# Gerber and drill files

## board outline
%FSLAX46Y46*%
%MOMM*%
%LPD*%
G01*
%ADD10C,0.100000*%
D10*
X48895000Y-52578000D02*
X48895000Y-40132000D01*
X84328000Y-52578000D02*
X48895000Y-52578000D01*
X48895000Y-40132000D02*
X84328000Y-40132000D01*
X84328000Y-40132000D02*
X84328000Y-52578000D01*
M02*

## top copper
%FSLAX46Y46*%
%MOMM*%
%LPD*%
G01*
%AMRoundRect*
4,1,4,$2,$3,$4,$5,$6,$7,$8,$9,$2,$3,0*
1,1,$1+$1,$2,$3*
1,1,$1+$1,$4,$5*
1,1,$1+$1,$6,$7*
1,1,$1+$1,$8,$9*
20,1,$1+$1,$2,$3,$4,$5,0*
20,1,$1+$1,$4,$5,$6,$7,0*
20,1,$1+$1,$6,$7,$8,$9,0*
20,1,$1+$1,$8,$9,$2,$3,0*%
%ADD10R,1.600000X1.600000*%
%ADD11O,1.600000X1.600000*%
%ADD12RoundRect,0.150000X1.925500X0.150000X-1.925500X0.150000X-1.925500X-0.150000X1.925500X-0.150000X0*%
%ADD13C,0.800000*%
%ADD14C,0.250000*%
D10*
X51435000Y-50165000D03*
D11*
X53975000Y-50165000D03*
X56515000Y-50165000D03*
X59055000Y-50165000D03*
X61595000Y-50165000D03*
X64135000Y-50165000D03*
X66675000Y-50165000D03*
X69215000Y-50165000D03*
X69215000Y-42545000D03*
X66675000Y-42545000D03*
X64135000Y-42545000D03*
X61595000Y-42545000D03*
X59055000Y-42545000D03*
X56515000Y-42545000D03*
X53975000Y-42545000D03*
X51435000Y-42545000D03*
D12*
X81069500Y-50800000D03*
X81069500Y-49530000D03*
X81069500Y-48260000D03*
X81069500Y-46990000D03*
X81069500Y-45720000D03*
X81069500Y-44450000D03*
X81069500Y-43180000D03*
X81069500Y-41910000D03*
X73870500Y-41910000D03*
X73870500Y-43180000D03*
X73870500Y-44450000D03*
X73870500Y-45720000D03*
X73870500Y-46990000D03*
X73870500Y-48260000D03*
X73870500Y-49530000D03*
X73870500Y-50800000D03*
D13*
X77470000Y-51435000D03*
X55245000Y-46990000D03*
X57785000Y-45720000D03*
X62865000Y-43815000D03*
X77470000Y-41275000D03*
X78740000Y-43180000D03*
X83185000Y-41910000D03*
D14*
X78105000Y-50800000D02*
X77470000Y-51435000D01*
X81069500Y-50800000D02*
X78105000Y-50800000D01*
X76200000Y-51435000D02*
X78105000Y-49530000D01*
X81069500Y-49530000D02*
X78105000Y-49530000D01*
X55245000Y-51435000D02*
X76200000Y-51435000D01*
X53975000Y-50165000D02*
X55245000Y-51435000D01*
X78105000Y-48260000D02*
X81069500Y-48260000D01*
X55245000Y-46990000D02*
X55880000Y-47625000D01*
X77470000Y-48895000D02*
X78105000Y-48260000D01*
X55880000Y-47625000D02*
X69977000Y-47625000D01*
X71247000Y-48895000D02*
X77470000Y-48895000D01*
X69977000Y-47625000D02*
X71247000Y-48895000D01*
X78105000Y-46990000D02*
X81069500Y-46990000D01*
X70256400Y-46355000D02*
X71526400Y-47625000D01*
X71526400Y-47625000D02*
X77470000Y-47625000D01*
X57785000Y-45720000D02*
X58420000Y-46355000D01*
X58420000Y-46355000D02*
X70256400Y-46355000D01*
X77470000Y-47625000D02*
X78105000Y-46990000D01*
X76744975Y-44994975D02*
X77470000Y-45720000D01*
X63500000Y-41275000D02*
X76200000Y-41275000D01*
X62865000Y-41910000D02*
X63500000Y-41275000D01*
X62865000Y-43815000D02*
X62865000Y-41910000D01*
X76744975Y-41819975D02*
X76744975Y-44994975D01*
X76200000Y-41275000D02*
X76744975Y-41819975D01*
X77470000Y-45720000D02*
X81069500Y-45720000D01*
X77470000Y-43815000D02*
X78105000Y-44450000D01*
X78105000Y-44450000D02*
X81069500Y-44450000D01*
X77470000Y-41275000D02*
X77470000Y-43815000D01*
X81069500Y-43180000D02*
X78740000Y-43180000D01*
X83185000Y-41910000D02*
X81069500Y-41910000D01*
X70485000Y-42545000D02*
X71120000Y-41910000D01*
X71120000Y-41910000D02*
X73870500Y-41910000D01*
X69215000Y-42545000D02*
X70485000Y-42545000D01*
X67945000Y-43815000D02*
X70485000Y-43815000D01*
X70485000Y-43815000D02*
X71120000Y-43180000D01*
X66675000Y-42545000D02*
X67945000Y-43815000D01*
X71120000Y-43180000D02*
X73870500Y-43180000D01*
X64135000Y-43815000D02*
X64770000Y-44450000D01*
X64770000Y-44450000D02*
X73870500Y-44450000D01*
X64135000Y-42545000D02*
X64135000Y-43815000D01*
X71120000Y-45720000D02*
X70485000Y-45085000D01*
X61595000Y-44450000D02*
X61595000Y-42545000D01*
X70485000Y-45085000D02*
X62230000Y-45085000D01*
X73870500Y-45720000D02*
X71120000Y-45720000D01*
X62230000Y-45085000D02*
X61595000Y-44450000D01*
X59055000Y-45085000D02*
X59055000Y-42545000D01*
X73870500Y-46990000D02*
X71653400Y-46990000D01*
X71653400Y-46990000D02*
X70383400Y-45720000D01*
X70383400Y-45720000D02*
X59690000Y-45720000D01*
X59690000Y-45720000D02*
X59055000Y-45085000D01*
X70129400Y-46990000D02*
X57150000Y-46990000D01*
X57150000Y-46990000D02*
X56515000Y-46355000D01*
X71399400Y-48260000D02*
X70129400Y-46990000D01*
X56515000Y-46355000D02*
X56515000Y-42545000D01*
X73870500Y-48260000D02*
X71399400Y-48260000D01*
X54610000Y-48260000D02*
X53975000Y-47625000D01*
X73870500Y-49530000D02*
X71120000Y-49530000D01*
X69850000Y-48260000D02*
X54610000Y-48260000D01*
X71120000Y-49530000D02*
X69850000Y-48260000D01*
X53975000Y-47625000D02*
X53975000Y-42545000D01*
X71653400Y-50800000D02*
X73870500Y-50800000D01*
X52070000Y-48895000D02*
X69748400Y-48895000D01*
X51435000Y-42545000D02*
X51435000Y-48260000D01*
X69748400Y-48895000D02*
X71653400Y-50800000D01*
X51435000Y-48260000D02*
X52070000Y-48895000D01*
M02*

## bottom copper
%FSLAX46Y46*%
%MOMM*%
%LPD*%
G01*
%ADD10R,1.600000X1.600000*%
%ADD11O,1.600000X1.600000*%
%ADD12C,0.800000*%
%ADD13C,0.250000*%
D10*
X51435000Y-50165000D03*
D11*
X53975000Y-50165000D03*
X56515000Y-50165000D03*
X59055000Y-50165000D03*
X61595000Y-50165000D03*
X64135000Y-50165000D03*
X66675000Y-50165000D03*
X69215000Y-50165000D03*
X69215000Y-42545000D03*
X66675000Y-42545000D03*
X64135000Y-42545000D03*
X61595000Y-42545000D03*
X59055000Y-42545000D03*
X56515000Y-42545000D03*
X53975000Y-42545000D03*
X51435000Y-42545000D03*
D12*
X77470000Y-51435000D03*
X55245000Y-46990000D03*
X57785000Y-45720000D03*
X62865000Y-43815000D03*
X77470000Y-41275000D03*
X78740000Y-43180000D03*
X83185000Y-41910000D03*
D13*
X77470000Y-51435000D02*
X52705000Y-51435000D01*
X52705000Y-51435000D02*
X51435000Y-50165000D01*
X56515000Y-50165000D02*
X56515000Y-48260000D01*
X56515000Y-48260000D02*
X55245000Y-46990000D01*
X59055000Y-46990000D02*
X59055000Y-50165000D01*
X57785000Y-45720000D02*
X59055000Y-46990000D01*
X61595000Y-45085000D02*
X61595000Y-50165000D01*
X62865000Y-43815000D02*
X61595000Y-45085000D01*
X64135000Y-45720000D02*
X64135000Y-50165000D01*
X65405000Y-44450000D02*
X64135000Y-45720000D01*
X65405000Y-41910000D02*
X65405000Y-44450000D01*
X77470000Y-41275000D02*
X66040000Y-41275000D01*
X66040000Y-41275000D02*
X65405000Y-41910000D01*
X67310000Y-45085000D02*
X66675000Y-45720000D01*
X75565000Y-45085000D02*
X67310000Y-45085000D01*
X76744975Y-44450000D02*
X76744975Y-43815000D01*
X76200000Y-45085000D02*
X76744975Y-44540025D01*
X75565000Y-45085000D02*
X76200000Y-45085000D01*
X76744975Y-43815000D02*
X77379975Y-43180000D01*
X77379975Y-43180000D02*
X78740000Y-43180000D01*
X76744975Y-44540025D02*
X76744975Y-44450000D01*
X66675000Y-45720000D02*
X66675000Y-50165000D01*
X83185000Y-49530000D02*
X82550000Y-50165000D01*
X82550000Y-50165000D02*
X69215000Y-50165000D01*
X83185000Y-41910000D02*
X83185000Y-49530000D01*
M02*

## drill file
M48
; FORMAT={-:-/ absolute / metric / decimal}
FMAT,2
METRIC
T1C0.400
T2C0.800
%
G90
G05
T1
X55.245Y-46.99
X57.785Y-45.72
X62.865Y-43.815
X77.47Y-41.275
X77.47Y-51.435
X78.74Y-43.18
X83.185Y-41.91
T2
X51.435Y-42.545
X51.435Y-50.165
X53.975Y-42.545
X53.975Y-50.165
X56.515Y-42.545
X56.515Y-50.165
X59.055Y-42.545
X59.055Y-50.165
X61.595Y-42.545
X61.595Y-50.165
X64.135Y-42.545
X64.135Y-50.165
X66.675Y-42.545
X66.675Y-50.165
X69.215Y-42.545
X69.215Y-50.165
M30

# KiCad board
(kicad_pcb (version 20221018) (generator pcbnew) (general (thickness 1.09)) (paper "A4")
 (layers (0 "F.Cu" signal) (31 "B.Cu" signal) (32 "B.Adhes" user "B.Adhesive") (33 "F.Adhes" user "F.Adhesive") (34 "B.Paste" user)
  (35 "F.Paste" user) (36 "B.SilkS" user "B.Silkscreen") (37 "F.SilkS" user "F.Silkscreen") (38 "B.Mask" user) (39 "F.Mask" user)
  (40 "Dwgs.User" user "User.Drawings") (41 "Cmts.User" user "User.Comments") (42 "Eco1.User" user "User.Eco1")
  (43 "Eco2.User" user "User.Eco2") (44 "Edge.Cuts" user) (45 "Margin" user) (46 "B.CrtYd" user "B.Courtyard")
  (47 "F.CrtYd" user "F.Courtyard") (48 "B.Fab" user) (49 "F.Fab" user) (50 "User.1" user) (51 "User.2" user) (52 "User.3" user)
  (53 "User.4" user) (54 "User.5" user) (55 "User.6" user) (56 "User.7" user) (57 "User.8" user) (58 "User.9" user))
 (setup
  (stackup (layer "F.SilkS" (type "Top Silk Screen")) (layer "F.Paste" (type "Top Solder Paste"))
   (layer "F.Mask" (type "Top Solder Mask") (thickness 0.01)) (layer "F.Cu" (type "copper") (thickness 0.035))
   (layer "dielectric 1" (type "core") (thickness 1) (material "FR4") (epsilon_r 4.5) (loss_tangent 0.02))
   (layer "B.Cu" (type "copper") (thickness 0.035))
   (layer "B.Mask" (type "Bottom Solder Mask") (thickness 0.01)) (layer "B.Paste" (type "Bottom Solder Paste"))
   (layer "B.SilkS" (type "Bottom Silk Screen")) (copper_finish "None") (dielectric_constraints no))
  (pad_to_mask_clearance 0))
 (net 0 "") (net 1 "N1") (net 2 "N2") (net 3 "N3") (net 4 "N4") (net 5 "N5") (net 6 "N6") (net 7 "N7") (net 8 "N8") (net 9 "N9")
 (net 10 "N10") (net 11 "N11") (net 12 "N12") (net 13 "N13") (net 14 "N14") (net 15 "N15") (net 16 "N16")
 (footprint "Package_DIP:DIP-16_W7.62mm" (layer "F.Cu") (at 51.435 50.165 90)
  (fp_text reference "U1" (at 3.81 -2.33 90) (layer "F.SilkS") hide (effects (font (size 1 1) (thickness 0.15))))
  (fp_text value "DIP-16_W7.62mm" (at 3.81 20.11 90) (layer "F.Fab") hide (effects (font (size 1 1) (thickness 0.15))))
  (pad "1" thru_hole rect (at 0 0 90) (size 1.6 1.6) (drill 0.8) (layers "*.Cu" "*.Mask") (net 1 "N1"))
  (pad "2" thru_hole oval (at 0 2.54 90) (size 1.6 1.6) (drill 0.8) (layers "*.Cu" "*.Mask") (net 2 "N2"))
  (pad "3" thru_hole oval (at 0 5.08 90) (size 1.6 1.6) (drill 0.8) (layers "*.Cu" "*.Mask") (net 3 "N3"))
  (pad "4" thru_hole oval (at 0 7.62 90) (size 1.6 1.6) (drill 0.8) (layers "*.Cu" "*.Mask") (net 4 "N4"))
  (pad "5" thru_hole oval (at 0 10.16 90) (size 1.6 1.6) (drill 0.8) (layers "*.Cu" "*.Mask") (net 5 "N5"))
  (pad "6" thru_hole oval (at 0 12.7 90) (size 1.6 1.6) (drill 0.8) (layers "*.Cu" "*.Mask") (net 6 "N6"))
  (pad "7" thru_hole oval (at 0 15.24 90) (size 1.6 1.6) (drill 0.8) (layers "*.Cu" "*.Mask") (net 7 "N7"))
  (pad "8" thru_hole oval (at 0 17.78 90) (size 1.6 1.6) (drill 0.8) (layers "*.Cu" "*.Mask") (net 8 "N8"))
  (pad "9" thru_hole oval (at 7.62 17.78 90) (size 1.6 1.6) (drill 0.8) (layers "*.Cu" "*.Mask") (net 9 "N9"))
  (pad "10" thru_hole oval (at 7.62 15.24 90) (size 1.6 1.6) (drill 0.8) (layers "*.Cu" "*.Mask") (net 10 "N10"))
  (pad "11" thru_hole oval (at 7.62 12.7 90) (size 1.6 1.6) (drill 0.8) (layers "*.Cu" "*.Mask") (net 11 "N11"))
  (pad "12" thru_hole oval (at 7.62 10.16 90) (size 1.6 1.6) (drill 0.8) (layers "*.Cu" "*.Mask") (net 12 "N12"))
  (pad "13" thru_hole oval (at 7.62 7.62 90) (size 1.6 1.6) (drill 0.8) (layers "*.Cu" "*.Mask") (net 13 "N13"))
  (pad "14" thru_hole oval (at 7.62 5.08 90) (size 1.6 1.6) (drill 0.8) (layers "*.Cu" "*.Mask") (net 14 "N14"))
  (pad "15" thru_hole oval (at 7.62 2.54 90) (size 1.6 1.6) (drill 0.8) (layers "*.Cu" "*.Mask") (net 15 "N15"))
  (pad "16" thru_hole oval (at 7.62 0 90) (size 1.6 1.6) (drill 0.8) (layers "*.Cu" "*.Mask") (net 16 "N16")))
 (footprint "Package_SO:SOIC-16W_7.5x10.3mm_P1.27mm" (layer "F.Cu") (at 77.47 46.355 180)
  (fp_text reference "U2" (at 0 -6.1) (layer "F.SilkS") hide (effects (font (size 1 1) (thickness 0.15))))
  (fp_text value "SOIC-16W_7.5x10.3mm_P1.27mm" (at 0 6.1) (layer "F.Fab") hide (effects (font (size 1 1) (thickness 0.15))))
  (pad "1" smd roundrect (at -3.5995 -4.445 180) (size 4.151 0.6) (layers "F.Cu" "F.Paste" "F.Mask") (roundrect_rratio 0.25) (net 1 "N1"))
  (pad "2" smd roundrect (at -3.5995 -3.175 180) (size 4.151 0.6) (layers "F.Cu" "F.Paste" "F.Mask") (roundrect_rratio 0.25) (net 2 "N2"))
  (pad "3" smd roundrect (at -3.5995 -1.905 180) (size 4.151 0.6) (layers "F.Cu" "F.Paste" "F.Mask") (roundrect_rratio 0.25) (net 3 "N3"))
  (pad "4" smd roundrect (at -3.5995 -0.635 180) (size 4.151 0.6) (layers "F.Cu" "F.Paste" "F.Mask") (roundrect_rratio 0.25) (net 4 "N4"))
  (pad "5" smd roundrect (at -3.5995 0.635 180) (size 4.151 0.6) (layers "F.Cu" "F.Paste" "F.Mask") (roundrect_rratio 0.25) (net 5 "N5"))
  (pad "6" smd roundrect (at -3.5995 1.905 180) (size 4.151 0.6) (layers "F.Cu" "F.Paste" "F.Mask") (roundrect_rratio 0.25) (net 6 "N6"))
  (pad "7" smd roundrect (at -3.5995 3.175 180) (size 4.151 0.6) (layers "F.Cu" "F.Paste" "F.Mask") (roundrect_rratio 0.25) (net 7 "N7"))
  (pad "8" smd roundrect (at -3.5995 4.445 180) (size 4.151 0.6) (layers "F.Cu" "F.Paste" "F.Mask") (roundrect_rratio 0.25) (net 8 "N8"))
  (pad "9" smd roundrect (at 3.5995 4.445 180) (size 4.151 0.6) (layers "F.Cu" "F.Paste" "F.Mask") (roundrect_rratio 0.25) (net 9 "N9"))
  (pad "10" smd roundrect (at 3.5995 3.175 180) (size 4.151 0.6) (layers "F.Cu" "F.Paste" "F.Mask") (roundrect_rratio 0.25) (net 10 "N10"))
  (pad "11" smd roundrect (at 3.5995 1.905 180) (size 4.151 0.6) (layers "F.Cu" "F.Paste" "F.Mask") (roundrect_rratio 0.25) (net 11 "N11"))
  (pad "12" smd roundrect (at 3.5995 0.635 180) (size 4.151 0.6) (layers "F.Cu" "F.Paste" "F.Mask") (roundrect_rratio 0.25) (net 12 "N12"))
  (pad "13" smd roundrect (at 3.5995 -0.635 180) (size 4.151 0.6) (layers "F.Cu" "F.Paste" "F.Mask") (roundrect_rratio 0.25) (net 13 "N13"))
  (pad "14" smd roundrect (at 3.5995 -1.905 180) (size 4.151 0.6) (layers "F.Cu" "F.Paste" "F.Mask") (roundrect_rratio 0.25) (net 14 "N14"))
  (pad "15" smd roundrect (at 3.5995 -3.175 180) (size 4.151 0.6) (layers "F.Cu" "F.Paste" "F.Mask") (roundrect_rratio 0.25) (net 15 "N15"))
  (pad "16" smd roundrect (at 3.5995 -4.445 180) (size 4.151 0.6) (layers "F.Cu" "F.Paste" "F.Mask") (roundrect_rratio 0.25) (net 16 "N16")))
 (gr_line (start 48.895 52.578) (end 48.895 40.132) (stroke (width 0.1) (type default)) (layer "Edge.Cuts"))
 (gr_line (start 84.328 52.578) (end 48.895 52.578) (stroke (width 0.1) (type default)) (layer "Edge.Cuts"))
 (gr_line (start 48.895 40.132) (end 84.328 40.132) (stroke (width 0.1) (type default)) (layer "Edge.Cuts"))
 (gr_line (start 84.328 40.132) (end 84.328 52.578) (stroke (width 0.1) (type default)) (layer "Edge.Cuts"))
 (segment (start 78.105 50.8) (end 77.47 51.435) (width 0.25) (layer "F.Cu") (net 1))
 (segment (start 81.0695 50.8) (end 78.105 50.8) (width 0.25) (layer "F.Cu") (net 1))
 (via (at 77.47 51.435) (size 0.8) (drill 0.4) (layers "F.Cu" "B.Cu") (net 1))
 (segment (start 77.47 51.435) (end 52.705 51.435) (width 0.25) (layer "B.Cu") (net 1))
 (segment (start 52.705 51.435) (end 51.435 50.165) (width 0.25) (layer "B.Cu") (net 1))
 (segment (start 76.2 51.435) (end 78.105 49.53) (width 0.25) (layer "F.Cu") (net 2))
 (segment (start 81.0695 49.53) (end 78.105 49.53) (width 0.25) (layer "F.Cu") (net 2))
 (segment (start 55.245 51.435) (end 76.2 51.435) (width 0.25) (layer "F.Cu") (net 2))
 (segment (start 53.975 50.165) (end 55.245 51.435) (width 0.25) (layer "F.Cu") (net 2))
 (segment (start 78.105 48.26) (end 81.0695 48.26) (width 0.25) (layer "F.Cu") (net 3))
 (segment (start 55.245 46.99) (end 55.88 47.625) (width 0.25) (layer "F.Cu") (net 3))
 (segment (start 77.47 48.895) (end 78.105 48.26) (width 0.25) (layer "F.Cu") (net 3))
 (segment (start 55.88 47.625) (end 69.977 47.625) (width 0.25) (layer "F.Cu") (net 3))
 (segment (start 71.247 48.895) (end 77.47 48.895) (width 0.25) (layer "F.Cu") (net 3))
 (segment (start 69.977 47.625) (end 71.247 48.895) (width 0.25) (layer "F.Cu") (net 3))
 (via (at 55.245 46.99) (size 0.8) (drill 0.4) (layers "F.Cu" "B.Cu") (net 3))
 (segment (start 56.515 50.165) (end 56.515 48.26) (width 0.25) (layer "B.Cu") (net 3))
 (segment (start 56.515 48.26) (end 55.245 46.99) (width 0.25) (layer "B.Cu") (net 3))
 (segment (start 78.105 46.99) (end 81.0695 46.99) (width 0.25) (layer "F.Cu") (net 4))
 (segment (start 70.2564 46.355) (end 71.5264 47.625) (width 0.25) (layer "F.Cu") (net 4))
 (segment (start 71.5264 47.625) (end 77.47 47.625) (width 0.25) (layer "F.Cu") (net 4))
 (segment (start 57.785 45.72) (end 58.42 46.355) (width 0.25) (layer "F.Cu") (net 4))
 (segment (start 58.42 46.355) (end 70.2564 46.355) (width 0.25) (layer "F.Cu") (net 4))
 (segment (start 77.47 47.625) (end 78.105 46.99) (width 0.25) (layer "F.Cu") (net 4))
 (via (at 57.785 45.72) (size 0.8) (drill 0.4) (layers "F.Cu" "B.Cu") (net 4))
 (segment (start 59.055 46.99) (end 59.055 50.165) (width 0.25) (layer "B.Cu") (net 4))
 (segment (start 57.785 45.72) (end 59.055 46.99) (width 0.25) (layer "B.Cu") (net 4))
 (segment (start 76.744975 44.994975) (end 77.47 45.72) (width 0.25) (layer "F.Cu") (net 5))
 (segment (start 63.5 41.275) (end 76.2 41.275) (width 0.25) (layer "F.Cu") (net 5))
 (segment (start 62.865 41.91) (end 63.5 41.275) (width 0.25) (layer "F.Cu") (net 5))
 (segment (start 62.865 43.815) (end 62.865 41.91) (width 0.25) (layer "F.Cu") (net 5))
 (segment (start 76.744975 41.819975) (end 76.744975 44.994975) (width 0.25) (layer "F.Cu") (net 5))
 (segment (start 76.2 41.275) (end 76.744975 41.819975) (width 0.25) (layer "F.Cu") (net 5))
 (segment (start 77.47 45.72) (end 81.0695 45.72) (width 0.25) (layer "F.Cu") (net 5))
 (via (at 62.865 43.815) (size 0.8) (drill 0.4) (layers "F.Cu" "B.Cu") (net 5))
 (segment (start 61.595 45.085) (end 61.595 50.165) (width 0.25) (layer "B.Cu") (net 5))
 (segment (start 62.865 43.815) (end 61.595 45.085) (width 0.25) (layer "B.Cu") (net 5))
 (segment (start 77.47 43.815) (end 78.105 44.45) (width 0.25) (layer "F.Cu") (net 6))
 (segment (start 78.105 44.45) (end 81.0695 44.45) (width 0.25) (layer "F.Cu") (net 6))
 (segment (start 77.47 41.275) (end 77.47 43.815) (width 0.25) (layer "F.Cu") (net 6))
 (via (at 77.47 41.275) (size 0.8) (drill 0.4) (layers "F.Cu" "B.Cu") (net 6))
 (segment (start 64.135 45.72) (end 64.135 50.165) (width 0.25) (layer "B.Cu") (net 6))
 (segment (start 65.405 44.45) (end 64.135 45.72) (width 0.25) (layer "B.Cu") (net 6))
 (segment (start 65.405 41.91) (end 65.405 44.45) (width 0.25) (layer "B.Cu") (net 6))
 (segment (start 77.47 41.275) (end 66.04 41.275) (width 0.25) (layer "B.Cu") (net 6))
 (segment (start 66.04 41.275) (end 65.405 41.91) (width 0.25) (layer "B.Cu") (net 6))
 (segment (start 81.0695 43.18) (end 78.74 43.18) (width 0.25) (layer "F.Cu") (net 7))
 (via (at 78.74 43.18) (size 0.8) (drill 0.4) (layers "F.Cu" "B.Cu") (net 7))
 (segment (start 67.31 45.085) (end 66.675 45.72) (width 0.25) (layer "B.Cu") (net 7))
 (segment (start 75.565 45.085) (end 67.31 45.085) (width 0.25) (layer "B.Cu") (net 7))
 (segment (start 76.744975 44.45) (end 76.744975 43.815) (width 0.25) (layer "B.Cu") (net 7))
 (segment (start 76.2 45.085) (end 76.744975 44.540025) (width 0.25) (layer "B.Cu") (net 7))
 (segment (start 75.565 45.085) (end 76.2 45.085) (width 0.25) (layer "B.Cu") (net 7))
 (segment (start 76.744975 43.815) (end 77.379975 43.18) (width 0.25) (layer "B.Cu") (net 7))
 (segment (start 77.379975 43.18) (end 78.74 43.18) (width 0.25) (layer "B.Cu") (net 7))
 (segment (start 76.744975 44.540025) (end 76.744975 44.45) (width 0.25) (layer "B.Cu") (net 7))
 (segment (start 66.675 45.72) (end 66.675 50.165) (width 0.25) (layer "B.Cu") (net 7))
 (segment (start 83.185 41.91) (end 81.0695 41.91) (width 0.25) (layer "F.Cu") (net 8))
 (via (at 83.185 41.91) (size 0.8) (drill 0.4) (layers "F.Cu" "B.Cu") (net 8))
 (segment (start 83.185 49.53) (end 82.55 50.165) (width 0.25) (layer "B.Cu") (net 8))
 (segment (start 82.55 50.165) (end 69.215 50.165) (width 0.25) (layer "B.Cu") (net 8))
 (segment (start 83.185 41.91) (end 83.185 49.53) (width 0.25) (layer "B.Cu") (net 8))
 (segment (start 70.485 42.545) (end 71.12 41.91) (width 0.25) (layer "F.Cu") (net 9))
 (segment (start 71.12 41.91) (end 73.8705 41.91) (width 0.25) (layer "F.Cu") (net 9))
 (segment (start 69.215 42.545) (end 70.485 42.545) (width 0.25) (layer "F.Cu") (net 9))
 (segment (start 67.945 43.815) (end 70.485 43.815) (width 0.25) (layer "F.Cu") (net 10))
 (segment (start 70.485 43.815) (end 71.12 43.18) (width 0.25) (layer "F.Cu") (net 10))
 (segment (start 66.675 42.545) (end 67.945 43.815) (width 0.25) (layer "F.Cu") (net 10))
 (segment (start 71.12 43.18) (end 73.8705 43.18) (width 0.25) (layer "F.Cu") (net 10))
 (segment (start 64.135 43.815) (end 64.77 44.45) (width 0.25) (layer "F.Cu") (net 11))
 (segment (start 64.77 44.45) (end 73.8705 44.45) (width 0.25) (layer "F.Cu") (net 11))
 (segment (start 64.135 42.545) (end 64.135 43.815) (width 0.25) (layer "F.Cu") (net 11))
 (segment (start 71.12 45.72) (end 70.485 45.085) (width 0.25) (layer "F.Cu") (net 12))
 (segment (start 61.595 44.45) (end 61.595 42.545) (width 0.25) (layer "F.Cu") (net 12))
 (segment (start 70.485 45.085) (end 62.23 45.085) (width 0.25) (layer "F.Cu") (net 12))
 (segment (start 73.8705 45.72) (end 71.12 45.72) (width 0.25) (layer "F.Cu") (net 12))
 (segment (start 62.23 45.085) (end 61.595 44.45) (width 0.25) (layer "F.Cu") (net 12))
 (segment (start 59.055 45.085) (end 59.055 42.545) (width 0.25) (layer "F.Cu") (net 13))
 (segment (start 73.8705 46.99) (end 71.6534 46.99) (width 0.25) (layer "F.Cu") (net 13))
 (segment (start 71.6534 46.99) (end 70.3834 45.72) (width 0.25) (layer "F.Cu") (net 13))
 (segment (start 70.3834 45.72) (end 59.69 45.72) (width 0.25) (layer "F.Cu") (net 13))
 (segment (start 59.69 45.72) (end 59.055 45.085) (width 0.25) (layer "F.Cu") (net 13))
 (segment (start 70.1294 46.99) (end 57.15 46.99) (width 0.25) (layer "F.Cu") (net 14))
 (segment (start 57.15 46.99) (end 56.515 46.355) (width 0.25) (layer "F.Cu") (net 14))
 (segment (start 71.3994 48.26) (end 70.1294 46.99) (width 0.25) (layer "F.Cu") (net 14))
 (segment (start 56.515 46.355) (end 56.515 42.545) (width 0.25) (layer "F.Cu") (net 14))
 (segment (start 73.8705 48.26) (end 71.3994 48.26) (width 0.25) (layer "F.Cu") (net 14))
 (segment (start 54.61 48.26) (end 53.975 47.625) (width 0.25) (layer "F.Cu") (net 15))
 (segment (start 73.8705 49.53) (end 71.12 49.53) (width 0.25) (layer "F.Cu") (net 15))
 (segment (start 69.85 48.26) (end 54.61 48.26) (width 0.25) (layer "F.Cu") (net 15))
 (segment (start 71.12 49.53) (end 69.85 48.26) (width 0.25) (layer "F.Cu") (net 15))
 (segment (start 53.975 47.625) (end 53.975 42.545) (width 0.25) (layer "F.Cu") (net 15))
 (segment (start 71.6534 50.8) (end 73.8705 50.8) (width 0.25) (layer "F.Cu") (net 16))
 (segment (start 52.07 48.895) (end 69.7484 48.895) (width 0.25) (layer "F.Cu") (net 16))
 (segment (start 51.435 42.545) (end 51.435 48.26) (width 0.25) (layer "F.Cu") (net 16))
 (segment (start 69.7484 48.895) (end 71.6534 50.8) (width 0.25) (layer "F.Cu") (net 16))
 (segment (start 51.435 48.26) (end 52.07 48.895) (width 0.25) (layer "F.Cu") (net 16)))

